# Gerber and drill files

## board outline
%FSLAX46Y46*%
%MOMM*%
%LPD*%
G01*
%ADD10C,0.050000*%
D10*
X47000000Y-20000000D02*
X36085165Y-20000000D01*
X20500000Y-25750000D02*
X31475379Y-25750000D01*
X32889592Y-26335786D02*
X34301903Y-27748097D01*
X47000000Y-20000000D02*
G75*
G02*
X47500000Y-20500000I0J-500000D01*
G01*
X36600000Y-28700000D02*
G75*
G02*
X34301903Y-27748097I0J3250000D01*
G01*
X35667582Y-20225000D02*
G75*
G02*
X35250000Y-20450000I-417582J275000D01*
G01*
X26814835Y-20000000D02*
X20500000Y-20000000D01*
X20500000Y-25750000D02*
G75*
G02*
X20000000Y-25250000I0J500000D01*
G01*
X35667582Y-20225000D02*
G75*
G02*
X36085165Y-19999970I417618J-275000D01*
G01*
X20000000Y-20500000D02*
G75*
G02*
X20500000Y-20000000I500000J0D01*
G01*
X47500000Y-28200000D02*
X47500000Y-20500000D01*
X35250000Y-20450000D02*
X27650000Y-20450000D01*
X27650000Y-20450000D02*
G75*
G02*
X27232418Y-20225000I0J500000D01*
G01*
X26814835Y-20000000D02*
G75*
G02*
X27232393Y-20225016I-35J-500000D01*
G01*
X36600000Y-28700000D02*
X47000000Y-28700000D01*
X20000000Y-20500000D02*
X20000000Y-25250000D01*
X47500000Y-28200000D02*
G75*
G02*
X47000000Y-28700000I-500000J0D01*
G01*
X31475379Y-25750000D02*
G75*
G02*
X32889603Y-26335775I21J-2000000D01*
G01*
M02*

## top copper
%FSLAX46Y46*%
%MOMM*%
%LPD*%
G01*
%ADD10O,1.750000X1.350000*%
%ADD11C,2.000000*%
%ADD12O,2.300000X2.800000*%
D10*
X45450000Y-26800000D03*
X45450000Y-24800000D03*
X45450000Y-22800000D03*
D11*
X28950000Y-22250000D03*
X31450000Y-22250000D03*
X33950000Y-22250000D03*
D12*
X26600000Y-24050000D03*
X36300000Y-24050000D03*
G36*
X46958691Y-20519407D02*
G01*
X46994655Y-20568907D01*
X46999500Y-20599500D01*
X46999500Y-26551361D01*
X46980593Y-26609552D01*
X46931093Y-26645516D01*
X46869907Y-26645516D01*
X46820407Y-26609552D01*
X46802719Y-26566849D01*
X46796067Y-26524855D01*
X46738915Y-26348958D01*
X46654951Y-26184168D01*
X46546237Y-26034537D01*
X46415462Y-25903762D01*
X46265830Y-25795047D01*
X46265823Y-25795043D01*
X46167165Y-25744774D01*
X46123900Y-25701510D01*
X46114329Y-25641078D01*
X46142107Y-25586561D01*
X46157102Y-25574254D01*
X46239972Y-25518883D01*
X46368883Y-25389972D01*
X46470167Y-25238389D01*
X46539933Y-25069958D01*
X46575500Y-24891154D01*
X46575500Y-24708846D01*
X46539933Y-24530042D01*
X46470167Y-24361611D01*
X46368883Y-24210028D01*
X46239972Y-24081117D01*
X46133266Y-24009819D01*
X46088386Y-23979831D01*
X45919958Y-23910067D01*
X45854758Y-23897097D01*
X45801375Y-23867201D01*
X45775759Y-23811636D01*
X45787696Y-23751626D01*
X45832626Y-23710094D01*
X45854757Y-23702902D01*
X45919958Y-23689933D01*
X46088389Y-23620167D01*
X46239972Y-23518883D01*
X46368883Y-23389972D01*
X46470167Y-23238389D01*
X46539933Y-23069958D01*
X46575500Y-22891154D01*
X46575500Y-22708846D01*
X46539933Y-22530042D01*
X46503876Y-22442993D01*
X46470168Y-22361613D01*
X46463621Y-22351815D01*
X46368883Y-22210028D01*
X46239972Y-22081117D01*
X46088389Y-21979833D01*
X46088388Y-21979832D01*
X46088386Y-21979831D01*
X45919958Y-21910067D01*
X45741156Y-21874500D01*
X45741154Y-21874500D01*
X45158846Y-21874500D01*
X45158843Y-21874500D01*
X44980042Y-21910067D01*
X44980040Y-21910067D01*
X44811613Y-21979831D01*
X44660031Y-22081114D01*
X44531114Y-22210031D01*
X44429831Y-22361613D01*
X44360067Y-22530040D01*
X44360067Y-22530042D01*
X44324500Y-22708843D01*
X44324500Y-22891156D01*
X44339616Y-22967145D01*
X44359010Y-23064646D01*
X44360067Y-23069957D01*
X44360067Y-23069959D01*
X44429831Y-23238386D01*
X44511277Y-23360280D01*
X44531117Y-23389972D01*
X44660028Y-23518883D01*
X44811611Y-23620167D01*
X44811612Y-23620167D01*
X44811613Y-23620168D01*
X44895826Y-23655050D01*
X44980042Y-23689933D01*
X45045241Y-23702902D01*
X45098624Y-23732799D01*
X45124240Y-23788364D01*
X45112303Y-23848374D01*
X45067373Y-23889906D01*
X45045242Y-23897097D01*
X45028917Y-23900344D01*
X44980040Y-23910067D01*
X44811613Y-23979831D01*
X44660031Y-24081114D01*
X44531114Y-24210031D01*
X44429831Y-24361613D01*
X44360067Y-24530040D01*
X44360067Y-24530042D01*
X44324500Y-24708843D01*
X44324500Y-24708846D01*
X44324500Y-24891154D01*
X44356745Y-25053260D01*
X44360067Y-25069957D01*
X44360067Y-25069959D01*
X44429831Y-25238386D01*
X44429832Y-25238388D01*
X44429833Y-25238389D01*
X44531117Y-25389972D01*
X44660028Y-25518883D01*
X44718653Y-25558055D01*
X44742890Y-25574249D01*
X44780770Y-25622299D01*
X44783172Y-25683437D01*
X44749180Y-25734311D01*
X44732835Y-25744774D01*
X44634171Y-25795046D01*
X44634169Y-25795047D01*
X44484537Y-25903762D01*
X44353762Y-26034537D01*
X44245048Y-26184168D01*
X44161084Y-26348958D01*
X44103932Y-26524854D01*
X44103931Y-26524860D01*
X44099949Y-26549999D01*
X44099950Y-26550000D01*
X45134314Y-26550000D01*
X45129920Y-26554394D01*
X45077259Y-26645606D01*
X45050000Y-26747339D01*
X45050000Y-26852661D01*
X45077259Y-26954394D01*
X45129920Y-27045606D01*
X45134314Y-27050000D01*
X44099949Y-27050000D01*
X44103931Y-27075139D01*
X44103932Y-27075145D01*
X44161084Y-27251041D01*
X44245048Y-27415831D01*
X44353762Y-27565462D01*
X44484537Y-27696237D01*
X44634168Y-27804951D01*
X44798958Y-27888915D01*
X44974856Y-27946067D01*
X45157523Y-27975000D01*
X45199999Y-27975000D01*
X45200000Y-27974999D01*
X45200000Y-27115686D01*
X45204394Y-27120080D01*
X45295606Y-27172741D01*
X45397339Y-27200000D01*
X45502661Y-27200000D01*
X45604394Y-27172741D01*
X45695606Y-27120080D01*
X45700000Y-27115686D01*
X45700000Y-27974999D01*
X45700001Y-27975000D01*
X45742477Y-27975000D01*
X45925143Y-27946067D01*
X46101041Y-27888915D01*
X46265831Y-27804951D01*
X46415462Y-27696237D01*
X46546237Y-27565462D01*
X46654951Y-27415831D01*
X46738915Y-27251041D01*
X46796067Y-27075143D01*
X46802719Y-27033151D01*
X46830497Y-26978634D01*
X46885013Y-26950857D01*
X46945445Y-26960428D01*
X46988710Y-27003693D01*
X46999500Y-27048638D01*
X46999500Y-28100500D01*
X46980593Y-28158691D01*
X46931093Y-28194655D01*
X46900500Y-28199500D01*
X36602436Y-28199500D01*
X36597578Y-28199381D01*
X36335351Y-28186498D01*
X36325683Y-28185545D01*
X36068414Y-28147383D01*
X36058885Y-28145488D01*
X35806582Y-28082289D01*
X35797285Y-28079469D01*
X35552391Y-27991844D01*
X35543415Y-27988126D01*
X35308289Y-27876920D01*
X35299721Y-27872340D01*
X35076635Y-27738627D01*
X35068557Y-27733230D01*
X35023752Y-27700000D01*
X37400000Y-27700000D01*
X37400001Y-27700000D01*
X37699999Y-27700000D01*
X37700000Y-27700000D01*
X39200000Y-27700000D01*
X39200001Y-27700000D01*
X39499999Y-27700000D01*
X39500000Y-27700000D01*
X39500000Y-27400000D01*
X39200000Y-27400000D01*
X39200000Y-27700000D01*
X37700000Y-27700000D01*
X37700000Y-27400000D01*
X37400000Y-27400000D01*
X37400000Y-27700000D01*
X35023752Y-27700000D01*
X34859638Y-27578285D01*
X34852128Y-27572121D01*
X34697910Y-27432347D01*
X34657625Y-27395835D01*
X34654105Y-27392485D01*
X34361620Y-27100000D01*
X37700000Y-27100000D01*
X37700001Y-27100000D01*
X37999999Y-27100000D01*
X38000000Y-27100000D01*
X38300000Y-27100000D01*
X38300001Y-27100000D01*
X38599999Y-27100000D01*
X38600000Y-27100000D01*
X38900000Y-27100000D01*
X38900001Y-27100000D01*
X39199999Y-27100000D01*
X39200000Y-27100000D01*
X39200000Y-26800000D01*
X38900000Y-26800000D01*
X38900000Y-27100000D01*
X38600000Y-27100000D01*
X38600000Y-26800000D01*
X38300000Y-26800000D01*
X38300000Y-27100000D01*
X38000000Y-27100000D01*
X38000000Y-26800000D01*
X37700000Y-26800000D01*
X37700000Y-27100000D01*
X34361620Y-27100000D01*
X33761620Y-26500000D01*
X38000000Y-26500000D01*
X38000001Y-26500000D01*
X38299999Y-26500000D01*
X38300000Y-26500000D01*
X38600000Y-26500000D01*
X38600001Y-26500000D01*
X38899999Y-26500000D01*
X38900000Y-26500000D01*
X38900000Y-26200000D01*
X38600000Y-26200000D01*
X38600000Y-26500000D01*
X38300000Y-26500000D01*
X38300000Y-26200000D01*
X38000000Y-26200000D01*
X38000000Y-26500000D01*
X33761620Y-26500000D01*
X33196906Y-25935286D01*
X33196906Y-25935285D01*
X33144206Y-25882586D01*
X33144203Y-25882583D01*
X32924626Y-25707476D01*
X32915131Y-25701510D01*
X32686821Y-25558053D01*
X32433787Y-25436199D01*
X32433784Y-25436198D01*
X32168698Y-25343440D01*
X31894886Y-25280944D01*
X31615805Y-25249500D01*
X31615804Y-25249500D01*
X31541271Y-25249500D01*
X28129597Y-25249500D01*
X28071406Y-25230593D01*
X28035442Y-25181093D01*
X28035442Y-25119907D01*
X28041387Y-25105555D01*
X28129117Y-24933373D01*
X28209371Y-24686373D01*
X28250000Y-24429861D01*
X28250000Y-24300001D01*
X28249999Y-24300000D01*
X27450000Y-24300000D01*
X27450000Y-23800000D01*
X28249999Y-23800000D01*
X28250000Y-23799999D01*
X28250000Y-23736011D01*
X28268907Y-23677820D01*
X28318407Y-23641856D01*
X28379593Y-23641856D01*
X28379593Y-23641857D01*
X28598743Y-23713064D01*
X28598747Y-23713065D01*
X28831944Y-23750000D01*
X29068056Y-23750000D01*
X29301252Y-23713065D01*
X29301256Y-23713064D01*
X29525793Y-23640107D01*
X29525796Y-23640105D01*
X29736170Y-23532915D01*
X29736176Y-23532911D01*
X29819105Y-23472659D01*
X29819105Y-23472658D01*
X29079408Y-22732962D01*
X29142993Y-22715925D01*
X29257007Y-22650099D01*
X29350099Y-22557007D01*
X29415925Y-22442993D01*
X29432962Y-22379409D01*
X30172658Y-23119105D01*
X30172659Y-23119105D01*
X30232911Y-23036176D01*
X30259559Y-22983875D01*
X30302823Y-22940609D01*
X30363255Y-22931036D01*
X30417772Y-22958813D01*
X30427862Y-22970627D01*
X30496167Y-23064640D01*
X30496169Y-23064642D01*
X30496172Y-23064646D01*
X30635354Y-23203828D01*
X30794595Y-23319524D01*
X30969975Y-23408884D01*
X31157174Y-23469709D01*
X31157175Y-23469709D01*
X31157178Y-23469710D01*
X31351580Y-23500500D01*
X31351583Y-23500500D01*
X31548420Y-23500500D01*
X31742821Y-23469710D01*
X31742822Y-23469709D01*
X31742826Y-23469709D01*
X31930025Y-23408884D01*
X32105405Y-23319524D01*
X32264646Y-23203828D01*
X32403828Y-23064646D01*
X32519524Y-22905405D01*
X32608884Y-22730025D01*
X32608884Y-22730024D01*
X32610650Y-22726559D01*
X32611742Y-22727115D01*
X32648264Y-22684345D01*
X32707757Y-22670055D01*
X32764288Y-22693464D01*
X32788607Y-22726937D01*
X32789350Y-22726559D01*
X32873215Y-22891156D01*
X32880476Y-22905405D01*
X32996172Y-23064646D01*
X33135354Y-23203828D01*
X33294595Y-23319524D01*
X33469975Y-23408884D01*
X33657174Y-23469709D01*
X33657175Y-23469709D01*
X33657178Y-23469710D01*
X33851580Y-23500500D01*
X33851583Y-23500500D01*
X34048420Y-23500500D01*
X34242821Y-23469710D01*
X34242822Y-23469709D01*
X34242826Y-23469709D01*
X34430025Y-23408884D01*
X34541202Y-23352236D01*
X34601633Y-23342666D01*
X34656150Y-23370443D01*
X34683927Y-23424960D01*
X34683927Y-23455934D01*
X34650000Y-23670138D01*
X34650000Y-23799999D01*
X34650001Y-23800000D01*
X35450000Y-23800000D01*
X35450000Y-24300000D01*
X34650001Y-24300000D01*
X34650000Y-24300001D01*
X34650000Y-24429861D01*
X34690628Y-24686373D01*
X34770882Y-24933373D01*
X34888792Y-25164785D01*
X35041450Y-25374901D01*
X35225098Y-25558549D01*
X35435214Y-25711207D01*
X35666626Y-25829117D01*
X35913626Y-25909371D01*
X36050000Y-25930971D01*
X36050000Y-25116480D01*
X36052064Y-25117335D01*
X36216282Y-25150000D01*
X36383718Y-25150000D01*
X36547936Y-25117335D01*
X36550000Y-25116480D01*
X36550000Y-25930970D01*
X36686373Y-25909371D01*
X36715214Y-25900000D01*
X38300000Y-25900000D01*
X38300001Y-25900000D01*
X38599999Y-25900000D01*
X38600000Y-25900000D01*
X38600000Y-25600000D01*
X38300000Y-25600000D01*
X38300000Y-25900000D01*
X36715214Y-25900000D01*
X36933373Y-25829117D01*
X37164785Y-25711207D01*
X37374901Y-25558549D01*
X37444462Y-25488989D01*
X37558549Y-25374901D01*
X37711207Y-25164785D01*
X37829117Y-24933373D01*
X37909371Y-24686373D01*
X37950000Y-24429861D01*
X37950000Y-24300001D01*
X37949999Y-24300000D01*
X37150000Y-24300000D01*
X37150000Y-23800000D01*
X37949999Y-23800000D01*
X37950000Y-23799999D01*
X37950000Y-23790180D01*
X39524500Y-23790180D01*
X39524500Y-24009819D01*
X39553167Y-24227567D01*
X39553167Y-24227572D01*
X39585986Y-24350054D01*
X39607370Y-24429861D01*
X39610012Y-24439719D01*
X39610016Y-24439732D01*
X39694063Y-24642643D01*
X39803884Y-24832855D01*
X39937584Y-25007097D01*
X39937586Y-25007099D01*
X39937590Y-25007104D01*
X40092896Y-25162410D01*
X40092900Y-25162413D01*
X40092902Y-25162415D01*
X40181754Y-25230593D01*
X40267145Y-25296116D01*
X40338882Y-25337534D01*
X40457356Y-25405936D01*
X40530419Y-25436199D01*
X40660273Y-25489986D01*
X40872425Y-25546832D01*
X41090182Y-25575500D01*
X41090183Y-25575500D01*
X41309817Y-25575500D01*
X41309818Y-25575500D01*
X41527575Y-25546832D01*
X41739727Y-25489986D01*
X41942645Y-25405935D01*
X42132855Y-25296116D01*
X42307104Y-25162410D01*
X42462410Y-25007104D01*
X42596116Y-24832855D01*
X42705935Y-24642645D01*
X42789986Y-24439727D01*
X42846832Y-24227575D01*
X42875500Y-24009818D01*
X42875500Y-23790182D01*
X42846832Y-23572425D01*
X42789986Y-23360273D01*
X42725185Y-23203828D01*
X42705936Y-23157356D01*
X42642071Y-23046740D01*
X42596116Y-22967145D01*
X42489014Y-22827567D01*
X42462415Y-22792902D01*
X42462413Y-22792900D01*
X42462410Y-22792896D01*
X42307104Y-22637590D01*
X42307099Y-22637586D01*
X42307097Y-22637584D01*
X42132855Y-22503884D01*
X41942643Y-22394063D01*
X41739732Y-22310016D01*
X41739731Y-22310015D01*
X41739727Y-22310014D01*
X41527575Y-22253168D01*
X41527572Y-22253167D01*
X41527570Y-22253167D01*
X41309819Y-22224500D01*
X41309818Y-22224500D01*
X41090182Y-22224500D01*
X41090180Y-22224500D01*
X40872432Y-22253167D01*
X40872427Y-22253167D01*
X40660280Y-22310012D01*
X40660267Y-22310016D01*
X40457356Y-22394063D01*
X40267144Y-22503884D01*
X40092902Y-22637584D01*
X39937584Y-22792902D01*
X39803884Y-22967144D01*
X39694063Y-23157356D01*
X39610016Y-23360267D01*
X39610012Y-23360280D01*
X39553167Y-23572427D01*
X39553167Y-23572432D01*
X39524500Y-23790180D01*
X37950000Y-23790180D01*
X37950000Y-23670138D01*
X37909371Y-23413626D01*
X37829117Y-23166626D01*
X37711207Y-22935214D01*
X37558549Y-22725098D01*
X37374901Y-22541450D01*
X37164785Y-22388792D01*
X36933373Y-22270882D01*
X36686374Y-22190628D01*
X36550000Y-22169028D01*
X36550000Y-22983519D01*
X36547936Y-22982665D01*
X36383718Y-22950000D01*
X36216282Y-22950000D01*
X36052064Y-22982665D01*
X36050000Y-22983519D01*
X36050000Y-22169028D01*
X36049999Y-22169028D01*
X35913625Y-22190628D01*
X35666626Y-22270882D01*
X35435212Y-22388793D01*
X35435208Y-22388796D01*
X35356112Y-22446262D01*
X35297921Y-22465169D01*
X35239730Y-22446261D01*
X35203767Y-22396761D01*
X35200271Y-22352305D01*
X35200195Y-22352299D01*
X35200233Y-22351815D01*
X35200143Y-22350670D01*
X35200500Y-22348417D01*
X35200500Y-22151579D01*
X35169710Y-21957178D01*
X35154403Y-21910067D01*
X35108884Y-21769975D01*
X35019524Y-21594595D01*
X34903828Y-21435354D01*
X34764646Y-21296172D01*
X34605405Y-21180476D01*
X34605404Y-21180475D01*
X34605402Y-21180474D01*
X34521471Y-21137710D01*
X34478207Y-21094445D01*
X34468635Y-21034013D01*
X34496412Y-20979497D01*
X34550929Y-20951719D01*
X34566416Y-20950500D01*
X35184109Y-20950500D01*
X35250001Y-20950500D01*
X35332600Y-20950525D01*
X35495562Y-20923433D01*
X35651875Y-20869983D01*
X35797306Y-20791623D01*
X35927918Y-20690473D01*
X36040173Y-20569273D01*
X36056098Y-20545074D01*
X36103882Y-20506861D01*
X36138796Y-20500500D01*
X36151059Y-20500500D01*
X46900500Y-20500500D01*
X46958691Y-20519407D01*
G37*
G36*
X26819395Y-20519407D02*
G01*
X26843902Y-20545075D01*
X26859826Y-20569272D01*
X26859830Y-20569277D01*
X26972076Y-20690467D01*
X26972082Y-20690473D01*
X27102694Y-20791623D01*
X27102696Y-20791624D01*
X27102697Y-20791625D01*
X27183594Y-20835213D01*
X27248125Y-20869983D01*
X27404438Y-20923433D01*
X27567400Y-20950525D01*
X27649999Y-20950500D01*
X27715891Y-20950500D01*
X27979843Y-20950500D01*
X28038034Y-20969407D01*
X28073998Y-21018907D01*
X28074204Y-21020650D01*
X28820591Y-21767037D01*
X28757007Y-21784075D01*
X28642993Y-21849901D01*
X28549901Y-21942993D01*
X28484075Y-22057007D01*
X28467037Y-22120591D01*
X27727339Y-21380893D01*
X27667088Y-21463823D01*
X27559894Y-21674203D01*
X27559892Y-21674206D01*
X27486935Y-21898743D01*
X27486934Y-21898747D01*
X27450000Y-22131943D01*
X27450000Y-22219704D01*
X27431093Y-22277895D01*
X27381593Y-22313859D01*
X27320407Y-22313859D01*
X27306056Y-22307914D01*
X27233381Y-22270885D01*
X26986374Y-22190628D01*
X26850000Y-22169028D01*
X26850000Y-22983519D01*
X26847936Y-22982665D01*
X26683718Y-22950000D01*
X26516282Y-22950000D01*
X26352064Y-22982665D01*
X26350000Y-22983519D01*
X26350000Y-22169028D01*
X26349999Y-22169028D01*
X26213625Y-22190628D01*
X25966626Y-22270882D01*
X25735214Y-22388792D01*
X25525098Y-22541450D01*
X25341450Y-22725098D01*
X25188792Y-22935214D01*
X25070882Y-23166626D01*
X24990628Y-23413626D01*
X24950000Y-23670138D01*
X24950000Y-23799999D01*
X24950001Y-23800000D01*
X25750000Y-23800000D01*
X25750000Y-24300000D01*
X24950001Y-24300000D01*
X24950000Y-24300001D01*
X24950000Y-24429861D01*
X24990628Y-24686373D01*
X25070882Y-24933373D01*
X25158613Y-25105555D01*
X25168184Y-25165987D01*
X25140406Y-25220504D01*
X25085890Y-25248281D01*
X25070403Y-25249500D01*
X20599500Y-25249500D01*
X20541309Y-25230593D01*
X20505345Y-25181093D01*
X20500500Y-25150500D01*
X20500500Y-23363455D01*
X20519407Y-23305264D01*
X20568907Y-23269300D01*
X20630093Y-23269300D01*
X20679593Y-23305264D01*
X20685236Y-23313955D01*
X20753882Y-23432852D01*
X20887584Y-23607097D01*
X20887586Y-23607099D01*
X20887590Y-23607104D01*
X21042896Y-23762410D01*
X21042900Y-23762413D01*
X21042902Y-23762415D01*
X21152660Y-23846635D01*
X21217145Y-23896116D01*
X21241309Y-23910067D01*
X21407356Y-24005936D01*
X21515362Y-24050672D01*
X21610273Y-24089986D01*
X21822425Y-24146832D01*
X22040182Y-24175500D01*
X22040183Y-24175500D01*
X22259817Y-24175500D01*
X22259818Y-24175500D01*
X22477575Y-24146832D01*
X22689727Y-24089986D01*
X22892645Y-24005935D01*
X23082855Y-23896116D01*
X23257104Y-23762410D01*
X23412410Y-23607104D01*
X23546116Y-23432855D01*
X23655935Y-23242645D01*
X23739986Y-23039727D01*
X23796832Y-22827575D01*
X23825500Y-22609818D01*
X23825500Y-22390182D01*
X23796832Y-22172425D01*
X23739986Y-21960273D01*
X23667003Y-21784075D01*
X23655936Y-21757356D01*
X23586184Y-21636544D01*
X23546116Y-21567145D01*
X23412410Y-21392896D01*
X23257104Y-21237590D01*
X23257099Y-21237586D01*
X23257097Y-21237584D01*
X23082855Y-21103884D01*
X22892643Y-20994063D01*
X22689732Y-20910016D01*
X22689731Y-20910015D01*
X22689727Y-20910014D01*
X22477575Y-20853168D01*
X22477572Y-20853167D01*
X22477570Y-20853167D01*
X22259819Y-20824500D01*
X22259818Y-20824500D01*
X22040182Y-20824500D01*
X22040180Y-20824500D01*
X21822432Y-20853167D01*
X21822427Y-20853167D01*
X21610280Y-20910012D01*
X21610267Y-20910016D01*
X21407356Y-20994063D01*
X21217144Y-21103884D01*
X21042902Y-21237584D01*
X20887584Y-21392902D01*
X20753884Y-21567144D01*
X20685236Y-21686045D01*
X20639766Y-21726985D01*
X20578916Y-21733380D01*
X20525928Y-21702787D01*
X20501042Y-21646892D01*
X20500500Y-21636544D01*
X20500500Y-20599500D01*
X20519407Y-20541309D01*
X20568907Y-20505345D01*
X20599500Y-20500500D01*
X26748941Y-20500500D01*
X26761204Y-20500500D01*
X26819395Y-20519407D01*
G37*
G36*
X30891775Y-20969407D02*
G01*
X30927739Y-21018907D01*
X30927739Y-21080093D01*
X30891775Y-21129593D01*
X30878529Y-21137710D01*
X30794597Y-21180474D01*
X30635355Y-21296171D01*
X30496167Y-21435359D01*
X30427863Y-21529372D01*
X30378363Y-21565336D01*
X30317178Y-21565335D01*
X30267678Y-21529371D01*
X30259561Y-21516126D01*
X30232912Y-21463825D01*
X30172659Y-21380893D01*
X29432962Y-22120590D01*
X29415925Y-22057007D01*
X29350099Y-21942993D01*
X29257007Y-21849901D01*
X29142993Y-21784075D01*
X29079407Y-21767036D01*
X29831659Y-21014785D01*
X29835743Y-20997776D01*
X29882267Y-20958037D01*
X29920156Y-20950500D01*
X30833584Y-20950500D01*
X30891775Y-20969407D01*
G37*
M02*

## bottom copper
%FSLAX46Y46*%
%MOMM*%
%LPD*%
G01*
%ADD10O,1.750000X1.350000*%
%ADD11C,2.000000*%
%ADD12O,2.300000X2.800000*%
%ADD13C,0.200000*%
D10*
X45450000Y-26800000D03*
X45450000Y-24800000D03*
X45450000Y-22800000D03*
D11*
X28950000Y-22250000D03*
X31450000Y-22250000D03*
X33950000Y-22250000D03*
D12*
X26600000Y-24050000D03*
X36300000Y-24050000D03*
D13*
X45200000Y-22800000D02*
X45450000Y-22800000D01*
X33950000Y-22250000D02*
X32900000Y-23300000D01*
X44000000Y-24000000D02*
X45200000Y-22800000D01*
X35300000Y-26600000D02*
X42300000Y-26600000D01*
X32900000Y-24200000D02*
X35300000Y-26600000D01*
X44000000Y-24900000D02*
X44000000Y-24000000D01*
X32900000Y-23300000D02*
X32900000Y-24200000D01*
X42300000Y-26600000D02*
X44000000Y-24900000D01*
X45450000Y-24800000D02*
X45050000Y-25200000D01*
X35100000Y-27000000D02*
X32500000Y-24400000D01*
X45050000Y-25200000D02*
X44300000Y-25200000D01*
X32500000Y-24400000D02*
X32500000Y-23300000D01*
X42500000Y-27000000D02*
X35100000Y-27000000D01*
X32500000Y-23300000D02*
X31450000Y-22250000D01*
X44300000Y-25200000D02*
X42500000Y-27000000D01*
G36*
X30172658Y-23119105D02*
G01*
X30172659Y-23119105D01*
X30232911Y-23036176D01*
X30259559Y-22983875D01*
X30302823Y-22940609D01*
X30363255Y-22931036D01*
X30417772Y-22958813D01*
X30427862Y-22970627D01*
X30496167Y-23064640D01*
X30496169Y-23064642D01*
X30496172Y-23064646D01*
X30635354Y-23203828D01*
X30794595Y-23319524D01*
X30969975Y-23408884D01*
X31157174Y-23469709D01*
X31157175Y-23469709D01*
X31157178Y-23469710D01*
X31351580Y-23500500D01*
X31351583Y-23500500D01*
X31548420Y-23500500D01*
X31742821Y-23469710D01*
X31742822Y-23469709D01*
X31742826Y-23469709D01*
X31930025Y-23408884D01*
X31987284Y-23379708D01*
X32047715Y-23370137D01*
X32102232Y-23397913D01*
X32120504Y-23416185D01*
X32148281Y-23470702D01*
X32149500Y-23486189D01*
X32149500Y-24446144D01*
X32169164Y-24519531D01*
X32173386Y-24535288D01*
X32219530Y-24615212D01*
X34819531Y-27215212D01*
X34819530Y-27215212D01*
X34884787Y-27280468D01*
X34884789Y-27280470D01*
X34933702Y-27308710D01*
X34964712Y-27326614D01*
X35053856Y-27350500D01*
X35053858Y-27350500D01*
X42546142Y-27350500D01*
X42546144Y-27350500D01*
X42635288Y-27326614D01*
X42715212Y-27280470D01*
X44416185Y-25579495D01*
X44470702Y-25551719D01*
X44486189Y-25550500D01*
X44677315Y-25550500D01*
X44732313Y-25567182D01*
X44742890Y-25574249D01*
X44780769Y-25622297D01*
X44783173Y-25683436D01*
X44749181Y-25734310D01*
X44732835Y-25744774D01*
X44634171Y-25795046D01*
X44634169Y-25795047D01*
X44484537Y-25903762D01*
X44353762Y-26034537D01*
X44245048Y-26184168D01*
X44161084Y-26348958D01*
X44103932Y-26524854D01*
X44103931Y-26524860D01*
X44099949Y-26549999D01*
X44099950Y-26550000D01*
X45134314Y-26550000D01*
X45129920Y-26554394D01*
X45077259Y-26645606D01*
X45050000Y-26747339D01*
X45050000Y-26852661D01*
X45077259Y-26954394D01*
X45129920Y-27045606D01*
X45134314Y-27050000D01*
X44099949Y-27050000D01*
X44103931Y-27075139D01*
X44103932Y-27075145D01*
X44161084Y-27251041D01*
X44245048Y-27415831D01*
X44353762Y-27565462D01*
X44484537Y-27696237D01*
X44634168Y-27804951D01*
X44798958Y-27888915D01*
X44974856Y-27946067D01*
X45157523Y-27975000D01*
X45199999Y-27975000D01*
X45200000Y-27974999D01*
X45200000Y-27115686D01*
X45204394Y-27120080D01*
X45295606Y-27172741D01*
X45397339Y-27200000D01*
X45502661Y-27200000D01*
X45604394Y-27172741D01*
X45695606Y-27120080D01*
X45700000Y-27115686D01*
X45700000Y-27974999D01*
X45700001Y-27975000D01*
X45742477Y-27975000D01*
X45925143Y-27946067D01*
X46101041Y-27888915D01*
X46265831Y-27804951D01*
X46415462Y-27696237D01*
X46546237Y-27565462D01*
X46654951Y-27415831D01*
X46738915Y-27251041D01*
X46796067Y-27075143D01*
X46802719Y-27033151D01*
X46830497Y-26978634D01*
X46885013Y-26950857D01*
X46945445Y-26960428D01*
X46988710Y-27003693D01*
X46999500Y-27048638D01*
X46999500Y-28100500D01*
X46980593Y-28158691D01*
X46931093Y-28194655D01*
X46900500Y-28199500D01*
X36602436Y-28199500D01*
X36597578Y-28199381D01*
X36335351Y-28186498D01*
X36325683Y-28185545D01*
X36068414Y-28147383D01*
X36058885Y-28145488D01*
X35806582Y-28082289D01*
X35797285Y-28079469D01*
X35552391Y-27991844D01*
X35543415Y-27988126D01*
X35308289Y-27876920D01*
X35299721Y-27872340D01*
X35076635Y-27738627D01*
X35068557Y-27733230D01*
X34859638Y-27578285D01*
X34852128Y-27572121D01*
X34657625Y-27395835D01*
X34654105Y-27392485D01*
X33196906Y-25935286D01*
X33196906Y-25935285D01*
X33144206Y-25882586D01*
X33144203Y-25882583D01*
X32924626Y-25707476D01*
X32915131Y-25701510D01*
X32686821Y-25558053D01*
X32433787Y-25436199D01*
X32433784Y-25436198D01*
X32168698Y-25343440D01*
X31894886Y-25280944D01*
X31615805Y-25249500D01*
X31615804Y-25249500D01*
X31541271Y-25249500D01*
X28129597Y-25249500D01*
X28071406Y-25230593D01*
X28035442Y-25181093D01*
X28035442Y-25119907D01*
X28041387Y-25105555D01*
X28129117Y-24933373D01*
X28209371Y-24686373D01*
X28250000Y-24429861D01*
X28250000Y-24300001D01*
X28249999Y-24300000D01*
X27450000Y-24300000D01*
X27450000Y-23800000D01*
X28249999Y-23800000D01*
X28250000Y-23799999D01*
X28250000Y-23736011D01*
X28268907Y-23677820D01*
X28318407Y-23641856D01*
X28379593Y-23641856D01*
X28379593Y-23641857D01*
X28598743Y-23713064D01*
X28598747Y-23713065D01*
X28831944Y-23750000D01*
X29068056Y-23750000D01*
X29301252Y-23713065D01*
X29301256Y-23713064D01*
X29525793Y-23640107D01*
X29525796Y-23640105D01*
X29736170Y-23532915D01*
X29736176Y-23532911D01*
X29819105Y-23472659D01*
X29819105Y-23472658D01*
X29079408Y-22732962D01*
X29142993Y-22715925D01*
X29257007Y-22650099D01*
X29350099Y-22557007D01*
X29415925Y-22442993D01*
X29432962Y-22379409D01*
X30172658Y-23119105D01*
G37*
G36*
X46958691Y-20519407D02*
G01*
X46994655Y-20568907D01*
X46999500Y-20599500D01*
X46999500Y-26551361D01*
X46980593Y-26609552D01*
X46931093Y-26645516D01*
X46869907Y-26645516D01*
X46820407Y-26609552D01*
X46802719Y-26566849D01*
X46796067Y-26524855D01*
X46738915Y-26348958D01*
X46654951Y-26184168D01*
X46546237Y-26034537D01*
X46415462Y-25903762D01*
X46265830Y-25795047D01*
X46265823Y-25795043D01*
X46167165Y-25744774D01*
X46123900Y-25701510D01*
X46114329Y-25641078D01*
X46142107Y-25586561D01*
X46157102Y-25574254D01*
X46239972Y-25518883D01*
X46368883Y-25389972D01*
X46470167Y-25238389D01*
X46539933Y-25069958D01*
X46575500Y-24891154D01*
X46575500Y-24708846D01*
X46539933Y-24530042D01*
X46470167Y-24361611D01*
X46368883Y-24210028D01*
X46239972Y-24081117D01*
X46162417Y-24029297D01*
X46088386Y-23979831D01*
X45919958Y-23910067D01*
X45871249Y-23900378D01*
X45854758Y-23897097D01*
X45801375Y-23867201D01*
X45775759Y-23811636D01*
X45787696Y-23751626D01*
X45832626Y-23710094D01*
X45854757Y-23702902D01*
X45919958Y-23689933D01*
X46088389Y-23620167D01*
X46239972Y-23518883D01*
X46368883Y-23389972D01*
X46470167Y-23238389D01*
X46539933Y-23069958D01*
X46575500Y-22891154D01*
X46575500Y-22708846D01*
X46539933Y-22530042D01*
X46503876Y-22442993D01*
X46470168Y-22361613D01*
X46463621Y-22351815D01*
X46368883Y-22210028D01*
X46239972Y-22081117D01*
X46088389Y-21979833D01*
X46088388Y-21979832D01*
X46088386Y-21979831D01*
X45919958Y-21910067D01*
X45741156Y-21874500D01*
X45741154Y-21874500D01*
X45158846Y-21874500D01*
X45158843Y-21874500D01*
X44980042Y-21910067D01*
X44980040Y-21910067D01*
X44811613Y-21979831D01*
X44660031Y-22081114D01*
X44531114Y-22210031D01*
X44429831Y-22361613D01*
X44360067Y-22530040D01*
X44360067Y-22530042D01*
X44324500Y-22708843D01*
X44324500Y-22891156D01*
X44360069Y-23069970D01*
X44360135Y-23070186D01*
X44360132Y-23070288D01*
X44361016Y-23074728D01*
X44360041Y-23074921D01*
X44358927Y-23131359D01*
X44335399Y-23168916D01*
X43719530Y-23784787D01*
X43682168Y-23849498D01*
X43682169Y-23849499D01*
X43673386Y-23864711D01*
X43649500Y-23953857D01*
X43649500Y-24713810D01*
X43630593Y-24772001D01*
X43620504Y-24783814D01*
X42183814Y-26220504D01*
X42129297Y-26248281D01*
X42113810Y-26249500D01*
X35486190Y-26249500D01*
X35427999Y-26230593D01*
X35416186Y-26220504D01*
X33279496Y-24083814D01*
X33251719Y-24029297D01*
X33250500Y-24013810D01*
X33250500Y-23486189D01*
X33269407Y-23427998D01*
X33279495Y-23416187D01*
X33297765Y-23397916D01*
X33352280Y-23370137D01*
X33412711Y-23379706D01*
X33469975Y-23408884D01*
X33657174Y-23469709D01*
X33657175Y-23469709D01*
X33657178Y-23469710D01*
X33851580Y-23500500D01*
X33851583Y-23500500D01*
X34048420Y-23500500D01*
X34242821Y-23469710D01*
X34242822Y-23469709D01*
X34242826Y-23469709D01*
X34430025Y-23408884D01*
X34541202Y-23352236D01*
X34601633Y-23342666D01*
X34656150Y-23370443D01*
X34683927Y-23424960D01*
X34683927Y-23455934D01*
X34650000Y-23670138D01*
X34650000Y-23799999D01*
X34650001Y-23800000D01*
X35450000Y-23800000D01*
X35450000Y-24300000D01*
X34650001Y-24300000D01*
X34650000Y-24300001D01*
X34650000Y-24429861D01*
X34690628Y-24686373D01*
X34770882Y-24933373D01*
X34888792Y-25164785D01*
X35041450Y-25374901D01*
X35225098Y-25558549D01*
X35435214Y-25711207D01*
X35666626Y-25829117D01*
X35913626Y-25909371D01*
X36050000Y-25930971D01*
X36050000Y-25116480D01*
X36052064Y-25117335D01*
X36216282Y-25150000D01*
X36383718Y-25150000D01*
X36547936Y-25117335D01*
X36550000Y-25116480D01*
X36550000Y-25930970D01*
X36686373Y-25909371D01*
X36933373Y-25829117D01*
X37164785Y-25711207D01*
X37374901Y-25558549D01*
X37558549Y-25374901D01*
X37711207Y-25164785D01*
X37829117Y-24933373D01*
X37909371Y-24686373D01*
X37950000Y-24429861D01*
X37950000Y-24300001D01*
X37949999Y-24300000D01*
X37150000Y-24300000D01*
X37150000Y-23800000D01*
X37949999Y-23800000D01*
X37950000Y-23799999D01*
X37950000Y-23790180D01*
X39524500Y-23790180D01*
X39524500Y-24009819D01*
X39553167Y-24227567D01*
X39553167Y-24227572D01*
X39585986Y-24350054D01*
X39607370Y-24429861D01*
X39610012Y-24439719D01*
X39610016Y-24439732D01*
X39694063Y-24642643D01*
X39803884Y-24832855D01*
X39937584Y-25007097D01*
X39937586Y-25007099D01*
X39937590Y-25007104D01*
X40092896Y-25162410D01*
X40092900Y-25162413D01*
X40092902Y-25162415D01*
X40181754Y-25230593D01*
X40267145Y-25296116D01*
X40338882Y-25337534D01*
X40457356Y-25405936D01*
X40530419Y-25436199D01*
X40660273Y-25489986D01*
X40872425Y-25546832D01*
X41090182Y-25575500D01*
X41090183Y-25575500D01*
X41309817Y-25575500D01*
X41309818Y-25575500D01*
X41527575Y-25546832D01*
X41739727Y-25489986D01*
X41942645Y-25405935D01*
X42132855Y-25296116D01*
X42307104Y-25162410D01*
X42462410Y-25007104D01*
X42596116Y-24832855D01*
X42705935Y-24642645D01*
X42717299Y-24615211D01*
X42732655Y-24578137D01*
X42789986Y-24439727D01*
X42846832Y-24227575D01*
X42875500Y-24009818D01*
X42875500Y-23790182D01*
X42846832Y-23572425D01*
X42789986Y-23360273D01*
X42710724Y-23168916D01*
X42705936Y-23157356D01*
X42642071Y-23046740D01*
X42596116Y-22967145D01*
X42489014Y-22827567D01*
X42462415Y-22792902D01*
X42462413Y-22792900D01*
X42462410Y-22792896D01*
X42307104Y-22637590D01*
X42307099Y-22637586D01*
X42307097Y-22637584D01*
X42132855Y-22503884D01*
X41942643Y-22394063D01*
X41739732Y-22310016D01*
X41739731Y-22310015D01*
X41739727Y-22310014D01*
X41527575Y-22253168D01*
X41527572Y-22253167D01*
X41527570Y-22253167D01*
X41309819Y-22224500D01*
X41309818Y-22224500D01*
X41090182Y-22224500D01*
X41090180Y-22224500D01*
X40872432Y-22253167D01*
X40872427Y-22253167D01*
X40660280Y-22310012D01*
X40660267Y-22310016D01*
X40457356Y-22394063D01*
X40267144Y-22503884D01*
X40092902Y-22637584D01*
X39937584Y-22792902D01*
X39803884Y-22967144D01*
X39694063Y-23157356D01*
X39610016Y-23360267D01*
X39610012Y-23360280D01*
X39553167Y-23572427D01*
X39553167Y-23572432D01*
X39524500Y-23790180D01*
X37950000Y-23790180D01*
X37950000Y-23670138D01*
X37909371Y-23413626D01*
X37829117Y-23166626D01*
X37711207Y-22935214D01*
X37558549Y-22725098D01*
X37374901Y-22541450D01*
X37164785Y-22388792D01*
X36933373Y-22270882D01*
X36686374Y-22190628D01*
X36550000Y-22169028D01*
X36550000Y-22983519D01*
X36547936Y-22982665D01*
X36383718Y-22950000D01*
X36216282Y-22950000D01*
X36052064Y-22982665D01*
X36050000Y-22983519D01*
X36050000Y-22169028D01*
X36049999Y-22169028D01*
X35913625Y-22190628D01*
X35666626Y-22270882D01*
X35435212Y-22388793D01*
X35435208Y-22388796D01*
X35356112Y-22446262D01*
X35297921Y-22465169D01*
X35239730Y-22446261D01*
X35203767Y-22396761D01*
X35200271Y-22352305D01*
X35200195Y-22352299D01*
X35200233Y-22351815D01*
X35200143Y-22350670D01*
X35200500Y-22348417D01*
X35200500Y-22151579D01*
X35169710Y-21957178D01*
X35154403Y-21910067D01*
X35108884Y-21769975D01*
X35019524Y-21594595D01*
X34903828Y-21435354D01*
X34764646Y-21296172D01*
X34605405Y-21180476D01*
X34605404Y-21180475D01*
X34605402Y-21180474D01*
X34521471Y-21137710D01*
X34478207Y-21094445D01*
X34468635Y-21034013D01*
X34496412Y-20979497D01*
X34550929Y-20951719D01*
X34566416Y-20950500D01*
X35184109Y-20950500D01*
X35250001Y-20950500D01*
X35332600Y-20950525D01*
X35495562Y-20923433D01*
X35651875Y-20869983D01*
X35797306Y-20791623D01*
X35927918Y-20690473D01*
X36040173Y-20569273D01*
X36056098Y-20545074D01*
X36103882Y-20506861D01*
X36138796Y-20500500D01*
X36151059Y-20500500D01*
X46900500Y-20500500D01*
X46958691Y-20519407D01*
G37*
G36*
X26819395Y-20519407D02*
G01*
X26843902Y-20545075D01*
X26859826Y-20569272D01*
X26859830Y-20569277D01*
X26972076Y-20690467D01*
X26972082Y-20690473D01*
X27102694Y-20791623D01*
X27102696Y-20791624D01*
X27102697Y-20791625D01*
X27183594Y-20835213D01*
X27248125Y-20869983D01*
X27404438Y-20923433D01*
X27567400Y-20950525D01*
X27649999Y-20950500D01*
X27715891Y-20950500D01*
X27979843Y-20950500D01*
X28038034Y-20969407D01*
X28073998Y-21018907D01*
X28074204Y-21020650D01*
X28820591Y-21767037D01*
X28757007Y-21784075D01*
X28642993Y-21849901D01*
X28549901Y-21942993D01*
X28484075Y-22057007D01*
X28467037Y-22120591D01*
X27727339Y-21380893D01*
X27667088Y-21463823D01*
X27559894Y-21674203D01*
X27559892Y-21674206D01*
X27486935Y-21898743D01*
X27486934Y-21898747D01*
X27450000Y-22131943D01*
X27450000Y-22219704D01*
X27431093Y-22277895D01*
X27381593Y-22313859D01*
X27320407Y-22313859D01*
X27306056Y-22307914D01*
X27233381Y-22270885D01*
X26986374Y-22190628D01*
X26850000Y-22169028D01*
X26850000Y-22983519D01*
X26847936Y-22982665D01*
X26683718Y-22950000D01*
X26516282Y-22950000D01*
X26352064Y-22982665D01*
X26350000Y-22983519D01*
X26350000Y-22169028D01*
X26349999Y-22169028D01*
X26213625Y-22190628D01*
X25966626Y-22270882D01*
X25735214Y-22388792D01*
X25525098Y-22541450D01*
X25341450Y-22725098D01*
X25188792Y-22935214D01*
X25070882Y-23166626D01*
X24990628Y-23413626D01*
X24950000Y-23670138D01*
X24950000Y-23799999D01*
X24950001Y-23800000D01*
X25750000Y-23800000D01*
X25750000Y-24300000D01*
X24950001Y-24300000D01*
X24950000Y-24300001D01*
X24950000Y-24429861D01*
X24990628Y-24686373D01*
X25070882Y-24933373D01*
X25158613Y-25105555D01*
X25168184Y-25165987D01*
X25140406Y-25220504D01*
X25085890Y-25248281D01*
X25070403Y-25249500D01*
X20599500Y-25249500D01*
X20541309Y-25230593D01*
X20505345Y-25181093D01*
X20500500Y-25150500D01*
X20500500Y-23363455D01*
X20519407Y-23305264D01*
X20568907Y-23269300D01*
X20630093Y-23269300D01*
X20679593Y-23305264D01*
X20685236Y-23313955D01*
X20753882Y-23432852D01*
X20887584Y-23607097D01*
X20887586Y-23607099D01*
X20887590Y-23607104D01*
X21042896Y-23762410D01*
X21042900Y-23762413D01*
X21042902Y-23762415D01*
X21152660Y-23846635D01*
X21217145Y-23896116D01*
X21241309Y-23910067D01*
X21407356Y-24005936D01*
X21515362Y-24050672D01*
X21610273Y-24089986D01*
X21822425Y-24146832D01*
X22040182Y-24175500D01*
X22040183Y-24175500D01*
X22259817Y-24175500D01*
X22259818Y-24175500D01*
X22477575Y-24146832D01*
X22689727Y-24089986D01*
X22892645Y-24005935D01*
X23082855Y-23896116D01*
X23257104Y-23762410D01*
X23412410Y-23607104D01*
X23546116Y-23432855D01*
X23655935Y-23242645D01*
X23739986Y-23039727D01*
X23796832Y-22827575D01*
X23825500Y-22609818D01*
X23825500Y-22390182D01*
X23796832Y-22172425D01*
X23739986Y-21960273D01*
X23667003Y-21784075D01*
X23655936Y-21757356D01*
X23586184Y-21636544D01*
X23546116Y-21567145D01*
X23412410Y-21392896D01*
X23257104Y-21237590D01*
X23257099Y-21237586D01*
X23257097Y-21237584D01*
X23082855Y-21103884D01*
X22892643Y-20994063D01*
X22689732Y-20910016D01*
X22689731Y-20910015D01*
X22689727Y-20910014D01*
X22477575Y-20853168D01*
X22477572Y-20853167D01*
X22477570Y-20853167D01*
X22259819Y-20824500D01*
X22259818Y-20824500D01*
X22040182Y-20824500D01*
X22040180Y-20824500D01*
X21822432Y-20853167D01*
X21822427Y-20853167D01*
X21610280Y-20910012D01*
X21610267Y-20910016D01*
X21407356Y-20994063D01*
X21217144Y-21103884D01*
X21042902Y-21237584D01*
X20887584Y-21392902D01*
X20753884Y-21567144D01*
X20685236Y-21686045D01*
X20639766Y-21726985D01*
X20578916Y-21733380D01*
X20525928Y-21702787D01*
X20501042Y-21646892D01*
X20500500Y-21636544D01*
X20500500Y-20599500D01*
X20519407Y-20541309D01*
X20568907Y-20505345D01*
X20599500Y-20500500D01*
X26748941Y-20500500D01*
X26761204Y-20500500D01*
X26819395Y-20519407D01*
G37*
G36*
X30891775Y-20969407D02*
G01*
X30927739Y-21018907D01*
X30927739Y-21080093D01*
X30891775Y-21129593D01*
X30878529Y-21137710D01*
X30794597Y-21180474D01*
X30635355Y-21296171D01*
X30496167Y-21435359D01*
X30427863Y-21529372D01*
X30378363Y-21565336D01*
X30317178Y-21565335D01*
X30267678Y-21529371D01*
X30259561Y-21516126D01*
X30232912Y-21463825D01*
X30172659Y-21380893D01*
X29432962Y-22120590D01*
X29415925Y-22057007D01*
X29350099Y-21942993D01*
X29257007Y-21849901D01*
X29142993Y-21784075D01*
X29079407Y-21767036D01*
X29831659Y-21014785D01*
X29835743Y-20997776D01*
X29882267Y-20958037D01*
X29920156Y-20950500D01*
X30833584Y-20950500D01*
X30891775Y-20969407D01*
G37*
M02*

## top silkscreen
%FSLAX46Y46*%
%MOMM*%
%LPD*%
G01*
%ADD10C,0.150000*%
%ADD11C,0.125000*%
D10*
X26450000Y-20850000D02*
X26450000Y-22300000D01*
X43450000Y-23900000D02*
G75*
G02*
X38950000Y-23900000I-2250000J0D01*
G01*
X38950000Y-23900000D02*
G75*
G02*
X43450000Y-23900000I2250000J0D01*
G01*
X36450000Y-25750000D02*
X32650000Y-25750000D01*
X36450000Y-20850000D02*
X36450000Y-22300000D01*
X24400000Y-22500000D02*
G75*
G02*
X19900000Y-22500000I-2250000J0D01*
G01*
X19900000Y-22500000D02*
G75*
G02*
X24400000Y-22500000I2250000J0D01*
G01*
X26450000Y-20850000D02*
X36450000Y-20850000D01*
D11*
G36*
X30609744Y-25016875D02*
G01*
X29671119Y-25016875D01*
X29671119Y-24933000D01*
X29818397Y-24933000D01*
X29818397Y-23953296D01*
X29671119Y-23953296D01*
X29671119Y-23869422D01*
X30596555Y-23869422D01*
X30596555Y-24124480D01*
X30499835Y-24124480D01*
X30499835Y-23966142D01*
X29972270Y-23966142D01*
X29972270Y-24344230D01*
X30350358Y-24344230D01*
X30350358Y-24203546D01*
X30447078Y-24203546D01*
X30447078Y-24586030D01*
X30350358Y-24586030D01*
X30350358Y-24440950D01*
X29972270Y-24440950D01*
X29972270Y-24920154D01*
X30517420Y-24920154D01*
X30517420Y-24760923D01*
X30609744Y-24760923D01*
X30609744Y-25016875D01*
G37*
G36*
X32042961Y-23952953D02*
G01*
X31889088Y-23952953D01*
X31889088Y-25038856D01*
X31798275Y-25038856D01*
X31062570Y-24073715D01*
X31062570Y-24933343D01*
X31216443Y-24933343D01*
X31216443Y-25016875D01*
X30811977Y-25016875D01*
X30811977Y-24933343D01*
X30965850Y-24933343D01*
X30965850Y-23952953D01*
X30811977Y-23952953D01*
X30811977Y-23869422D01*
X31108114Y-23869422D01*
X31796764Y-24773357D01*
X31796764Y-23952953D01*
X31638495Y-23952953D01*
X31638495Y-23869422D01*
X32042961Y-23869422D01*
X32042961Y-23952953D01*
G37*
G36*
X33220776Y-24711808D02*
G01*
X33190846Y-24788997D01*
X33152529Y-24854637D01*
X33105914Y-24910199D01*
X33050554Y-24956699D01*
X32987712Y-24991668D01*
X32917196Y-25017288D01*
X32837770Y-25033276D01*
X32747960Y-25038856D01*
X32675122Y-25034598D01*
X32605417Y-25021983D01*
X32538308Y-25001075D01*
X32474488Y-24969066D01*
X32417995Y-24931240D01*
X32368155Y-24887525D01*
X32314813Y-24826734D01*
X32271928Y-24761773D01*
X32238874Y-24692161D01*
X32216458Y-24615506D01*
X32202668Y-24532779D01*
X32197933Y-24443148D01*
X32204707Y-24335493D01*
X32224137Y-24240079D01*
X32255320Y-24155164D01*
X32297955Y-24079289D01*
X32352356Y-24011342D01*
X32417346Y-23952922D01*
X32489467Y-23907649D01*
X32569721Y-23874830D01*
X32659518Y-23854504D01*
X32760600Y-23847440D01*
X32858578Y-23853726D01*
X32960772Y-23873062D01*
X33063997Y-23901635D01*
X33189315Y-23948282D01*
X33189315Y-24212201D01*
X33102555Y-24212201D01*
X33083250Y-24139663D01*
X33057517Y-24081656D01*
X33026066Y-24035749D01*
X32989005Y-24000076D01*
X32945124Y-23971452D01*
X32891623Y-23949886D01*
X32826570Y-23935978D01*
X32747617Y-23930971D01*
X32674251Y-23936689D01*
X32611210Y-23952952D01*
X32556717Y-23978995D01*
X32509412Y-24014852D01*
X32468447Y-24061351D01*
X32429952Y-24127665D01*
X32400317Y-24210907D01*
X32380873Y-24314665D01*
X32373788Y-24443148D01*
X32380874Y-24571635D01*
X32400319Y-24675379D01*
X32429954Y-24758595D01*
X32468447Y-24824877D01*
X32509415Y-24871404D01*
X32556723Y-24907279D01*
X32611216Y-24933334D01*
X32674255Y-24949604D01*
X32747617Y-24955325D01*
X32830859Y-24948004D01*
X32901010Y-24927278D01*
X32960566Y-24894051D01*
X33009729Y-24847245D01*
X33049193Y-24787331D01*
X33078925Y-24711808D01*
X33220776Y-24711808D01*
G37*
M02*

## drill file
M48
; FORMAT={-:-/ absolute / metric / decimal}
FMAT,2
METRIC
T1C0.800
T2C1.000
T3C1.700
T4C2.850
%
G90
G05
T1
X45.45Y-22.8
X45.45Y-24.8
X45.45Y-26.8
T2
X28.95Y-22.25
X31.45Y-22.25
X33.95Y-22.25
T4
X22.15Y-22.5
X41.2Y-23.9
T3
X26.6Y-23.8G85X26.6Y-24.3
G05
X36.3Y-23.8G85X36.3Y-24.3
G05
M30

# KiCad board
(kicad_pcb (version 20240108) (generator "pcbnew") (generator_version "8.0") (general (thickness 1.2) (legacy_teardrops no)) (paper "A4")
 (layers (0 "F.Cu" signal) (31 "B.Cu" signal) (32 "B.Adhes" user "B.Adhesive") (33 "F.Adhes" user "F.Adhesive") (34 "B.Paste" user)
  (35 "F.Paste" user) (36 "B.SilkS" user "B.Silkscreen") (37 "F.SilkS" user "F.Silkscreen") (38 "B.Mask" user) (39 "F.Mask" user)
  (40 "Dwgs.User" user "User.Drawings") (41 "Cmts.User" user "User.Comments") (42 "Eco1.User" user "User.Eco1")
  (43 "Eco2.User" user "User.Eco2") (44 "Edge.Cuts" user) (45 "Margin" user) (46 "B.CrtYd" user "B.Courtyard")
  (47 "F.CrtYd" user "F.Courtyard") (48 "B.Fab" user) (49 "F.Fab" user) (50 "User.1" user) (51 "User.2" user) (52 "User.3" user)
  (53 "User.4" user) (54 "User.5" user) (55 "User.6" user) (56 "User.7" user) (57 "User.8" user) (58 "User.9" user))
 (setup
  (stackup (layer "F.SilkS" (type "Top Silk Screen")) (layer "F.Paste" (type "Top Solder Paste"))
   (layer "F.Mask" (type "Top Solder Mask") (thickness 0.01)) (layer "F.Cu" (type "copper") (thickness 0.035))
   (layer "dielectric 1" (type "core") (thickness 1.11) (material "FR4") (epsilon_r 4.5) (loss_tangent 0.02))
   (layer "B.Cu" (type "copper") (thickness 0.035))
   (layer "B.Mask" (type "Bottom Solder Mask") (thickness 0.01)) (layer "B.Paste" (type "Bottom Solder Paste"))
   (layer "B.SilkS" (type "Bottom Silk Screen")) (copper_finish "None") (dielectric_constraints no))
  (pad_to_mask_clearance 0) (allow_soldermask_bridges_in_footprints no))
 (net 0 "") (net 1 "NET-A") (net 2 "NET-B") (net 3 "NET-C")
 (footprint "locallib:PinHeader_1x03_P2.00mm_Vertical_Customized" (layer "F.Cu") (at 45.45 26.8 180)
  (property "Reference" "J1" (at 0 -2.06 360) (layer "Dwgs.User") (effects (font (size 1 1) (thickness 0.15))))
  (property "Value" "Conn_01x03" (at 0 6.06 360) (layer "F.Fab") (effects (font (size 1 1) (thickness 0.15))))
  (pad "1" thru_hole oval (at 0 0 180) (size 1.75 1.35) (drill 0.8) (layers "*.Cu" "F.Mask") (remove_unused_layers no) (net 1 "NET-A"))
  (pad "2" thru_hole oval (at 0 2 180) (size 1.75 1.35) (drill 0.8) (layers "*.Cu" "F.Mask") (remove_unused_layers no) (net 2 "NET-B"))
  (pad "3" thru_hole oval (at 0 4 180) (size 1.75 1.35) (drill 0.8) (layers "*.Cu" "F.Mask") (remove_unused_layers no) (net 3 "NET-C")))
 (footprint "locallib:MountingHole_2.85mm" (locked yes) (layer "F.Cu") (at 22.15 22.5)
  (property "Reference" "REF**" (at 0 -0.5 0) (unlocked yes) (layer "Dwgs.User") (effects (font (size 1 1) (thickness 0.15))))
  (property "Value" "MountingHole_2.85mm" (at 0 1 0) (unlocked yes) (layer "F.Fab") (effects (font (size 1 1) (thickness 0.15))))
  (pad "" np_thru_hole circle (at 0 0) (size 2.85 2.85) (drill 2.85) (layers "F&B.Cu" "*.Mask")))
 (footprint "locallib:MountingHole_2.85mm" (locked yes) (layer "F.Cu") (at 41.2 23.9)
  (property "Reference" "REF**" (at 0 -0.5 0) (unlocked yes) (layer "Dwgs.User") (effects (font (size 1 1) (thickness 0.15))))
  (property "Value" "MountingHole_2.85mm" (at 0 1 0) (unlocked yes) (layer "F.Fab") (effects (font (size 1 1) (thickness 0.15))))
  (pad "" np_thru_hole circle (at 0 0) (size 2.85 2.85) (drill 2.85) (layers "F&B.Cu" "*.Mask")))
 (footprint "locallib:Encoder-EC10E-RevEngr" (layer "F.Cu") (at 31.45 22.25)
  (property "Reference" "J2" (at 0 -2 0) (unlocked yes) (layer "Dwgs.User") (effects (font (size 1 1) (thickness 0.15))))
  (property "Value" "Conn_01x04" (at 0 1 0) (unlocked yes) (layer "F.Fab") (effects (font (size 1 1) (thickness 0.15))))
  (pad "1" thru_hole circle (at -2.5 0) (size 2 2) (drill 1) (layers "*.Cu" "B.Mask") (remove_unused_layers no) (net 1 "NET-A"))
  (pad "2" thru_hole circle (at 0 0) (size 2 2) (drill 1) (layers "*.Cu" "B.Mask") (remove_unused_layers no) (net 2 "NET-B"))
  (pad "3" thru_hole circle (at 2.5 0) (size 2 2) (drill 1) (layers "*.Cu" "B.Mask") (remove_unused_layers no) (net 3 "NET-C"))
  (pad "4" thru_hole oval (at -4.85 1.8) (size 2.3 2.8) (drill oval 1.7 2.2) (layers "*.Cu" "*.Mask") (remove_unused_layers no)
   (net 1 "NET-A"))
  (pad "4" thru_hole oval (at 4.85 1.8) (size 2.3 2.8) (drill oval 1.7 2.2) (layers "*.Cu" "*.Mask") (remove_unused_layers no)
   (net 1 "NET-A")))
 (gr_line (start 26.45 20.85) (end 26.45 22.3) (stroke (width 0.15) (type default)) (layer "F.SilkS"))
 (gr_circle (center 41.2 23.9) (end 43.45 23.9) (stroke (width 0.15) (type default)) (fill none) (layer "F.SilkS"))
 (gr_line (start 36.45 25.75) (end 32.65 25.75) (stroke (width 0.15) (type default)) (layer "F.SilkS"))
 (gr_line (start 36.45 20.85) (end 36.45 22.3) (stroke (width 0.15) (type default)) (layer "F.SilkS"))
 (gr_circle (center 22.15 22.5) (end 24.4 22.5) (stroke (width 0.15) (type default)) (fill none) (layer "F.SilkS"))
 (gr_line (start 26.45 20.85) (end 36.45 20.85) (stroke (width 0.15) (type default)) (layer "F.SilkS"))
 (gr_line (start 47 20) (end 36.085165 20) (stroke (width 0.05) (type default)) (layer "Edge.Cuts"))
 (gr_line (start 20.5 25.75) (end 31.475379 25.75) (stroke (width 0.05) (type default)) (layer "Edge.Cuts"))
 (gr_line (start 32.889592 26.335786) (end 34.301903 27.748097) (stroke (width 0.05) (type default)) (layer "Edge.Cuts"))
 (gr_arc (start 47 20) (mid 47.353553 20.146447) (end 47.5 20.5) (stroke (width 0.05) (type default)) (layer "Edge.Cuts"))
 (gr_arc (start 36.6 28.7) (mid 35.356279 28.452608) (end 34.301903 27.748097) (stroke (width 0.05) (type default)) (layer "Edge.Cuts"))
 (gr_arc (start 35.667582 20.225) (mid 35.487171 20.39017) (end 35.25 20.45) (stroke (width 0.05) (type default)) (layer "Edge.Cuts"))
 (gr_line (start 26.814835 20) (end 20.5 20) (stroke (width 0.05) (type default)) (layer "Edge.Cuts"))
 (gr_arc (start 20.5 25.75) (mid 20.146447 25.603553) (end 20 25.25) (stroke (width 0.05) (type default)) (layer "Edge.Cuts"))
 (gr_arc (start 35.667582 20.225) (mid 35.847994 20.05983) (end 36.085165 20) (stroke (width 0.05) (type default)) (layer "Edge.Cuts"))
 (gr_arc (start 20 20.5) (mid 20.146447 20.146447) (end 20.5 20) (stroke (width 0.05) (type default)) (layer "Edge.Cuts"))
 (gr_line (start 47.5 28.2) (end 47.5 20.5) (stroke (width 0.05) (type default)) (layer "Edge.Cuts"))
 (gr_line (start 35.25 20.45) (end 27.65 20.45) (stroke (width 0.05) (type default)) (layer "Edge.Cuts"))
 (gr_arc (start 27.65 20.45) (mid 27.412829 20.39017) (end 27.232418 20.225) (stroke (width 0.05) (type default)) (layer "Edge.Cuts"))
 (gr_arc (start 26.814835 20) (mid 27.052006 20.05983) (end 27.232418 20.225) (stroke (width 0.05) (type default)) (layer "Edge.Cuts"))
 (gr_line (start 36.6 28.7) (end 47 28.7) (stroke (width 0.05) (type default)) (layer "Edge.Cuts"))
 (gr_line (start 20 20.5) (end 20 25.25) (stroke (width 0.05) (type default)) (layer "Edge.Cuts"))
 (gr_arc (start 47.5 28.2) (mid 47.353553 28.553553) (end 47 28.7) (stroke (width 0.05) (type default)) (layer "Edge.Cuts"))
 (gr_arc (start 31.475379 25.75) (mid 32.240746 25.902241) (end 32.889592 26.335786) (stroke (width 0.05) (type default))
  (layer "Edge.Cuts"))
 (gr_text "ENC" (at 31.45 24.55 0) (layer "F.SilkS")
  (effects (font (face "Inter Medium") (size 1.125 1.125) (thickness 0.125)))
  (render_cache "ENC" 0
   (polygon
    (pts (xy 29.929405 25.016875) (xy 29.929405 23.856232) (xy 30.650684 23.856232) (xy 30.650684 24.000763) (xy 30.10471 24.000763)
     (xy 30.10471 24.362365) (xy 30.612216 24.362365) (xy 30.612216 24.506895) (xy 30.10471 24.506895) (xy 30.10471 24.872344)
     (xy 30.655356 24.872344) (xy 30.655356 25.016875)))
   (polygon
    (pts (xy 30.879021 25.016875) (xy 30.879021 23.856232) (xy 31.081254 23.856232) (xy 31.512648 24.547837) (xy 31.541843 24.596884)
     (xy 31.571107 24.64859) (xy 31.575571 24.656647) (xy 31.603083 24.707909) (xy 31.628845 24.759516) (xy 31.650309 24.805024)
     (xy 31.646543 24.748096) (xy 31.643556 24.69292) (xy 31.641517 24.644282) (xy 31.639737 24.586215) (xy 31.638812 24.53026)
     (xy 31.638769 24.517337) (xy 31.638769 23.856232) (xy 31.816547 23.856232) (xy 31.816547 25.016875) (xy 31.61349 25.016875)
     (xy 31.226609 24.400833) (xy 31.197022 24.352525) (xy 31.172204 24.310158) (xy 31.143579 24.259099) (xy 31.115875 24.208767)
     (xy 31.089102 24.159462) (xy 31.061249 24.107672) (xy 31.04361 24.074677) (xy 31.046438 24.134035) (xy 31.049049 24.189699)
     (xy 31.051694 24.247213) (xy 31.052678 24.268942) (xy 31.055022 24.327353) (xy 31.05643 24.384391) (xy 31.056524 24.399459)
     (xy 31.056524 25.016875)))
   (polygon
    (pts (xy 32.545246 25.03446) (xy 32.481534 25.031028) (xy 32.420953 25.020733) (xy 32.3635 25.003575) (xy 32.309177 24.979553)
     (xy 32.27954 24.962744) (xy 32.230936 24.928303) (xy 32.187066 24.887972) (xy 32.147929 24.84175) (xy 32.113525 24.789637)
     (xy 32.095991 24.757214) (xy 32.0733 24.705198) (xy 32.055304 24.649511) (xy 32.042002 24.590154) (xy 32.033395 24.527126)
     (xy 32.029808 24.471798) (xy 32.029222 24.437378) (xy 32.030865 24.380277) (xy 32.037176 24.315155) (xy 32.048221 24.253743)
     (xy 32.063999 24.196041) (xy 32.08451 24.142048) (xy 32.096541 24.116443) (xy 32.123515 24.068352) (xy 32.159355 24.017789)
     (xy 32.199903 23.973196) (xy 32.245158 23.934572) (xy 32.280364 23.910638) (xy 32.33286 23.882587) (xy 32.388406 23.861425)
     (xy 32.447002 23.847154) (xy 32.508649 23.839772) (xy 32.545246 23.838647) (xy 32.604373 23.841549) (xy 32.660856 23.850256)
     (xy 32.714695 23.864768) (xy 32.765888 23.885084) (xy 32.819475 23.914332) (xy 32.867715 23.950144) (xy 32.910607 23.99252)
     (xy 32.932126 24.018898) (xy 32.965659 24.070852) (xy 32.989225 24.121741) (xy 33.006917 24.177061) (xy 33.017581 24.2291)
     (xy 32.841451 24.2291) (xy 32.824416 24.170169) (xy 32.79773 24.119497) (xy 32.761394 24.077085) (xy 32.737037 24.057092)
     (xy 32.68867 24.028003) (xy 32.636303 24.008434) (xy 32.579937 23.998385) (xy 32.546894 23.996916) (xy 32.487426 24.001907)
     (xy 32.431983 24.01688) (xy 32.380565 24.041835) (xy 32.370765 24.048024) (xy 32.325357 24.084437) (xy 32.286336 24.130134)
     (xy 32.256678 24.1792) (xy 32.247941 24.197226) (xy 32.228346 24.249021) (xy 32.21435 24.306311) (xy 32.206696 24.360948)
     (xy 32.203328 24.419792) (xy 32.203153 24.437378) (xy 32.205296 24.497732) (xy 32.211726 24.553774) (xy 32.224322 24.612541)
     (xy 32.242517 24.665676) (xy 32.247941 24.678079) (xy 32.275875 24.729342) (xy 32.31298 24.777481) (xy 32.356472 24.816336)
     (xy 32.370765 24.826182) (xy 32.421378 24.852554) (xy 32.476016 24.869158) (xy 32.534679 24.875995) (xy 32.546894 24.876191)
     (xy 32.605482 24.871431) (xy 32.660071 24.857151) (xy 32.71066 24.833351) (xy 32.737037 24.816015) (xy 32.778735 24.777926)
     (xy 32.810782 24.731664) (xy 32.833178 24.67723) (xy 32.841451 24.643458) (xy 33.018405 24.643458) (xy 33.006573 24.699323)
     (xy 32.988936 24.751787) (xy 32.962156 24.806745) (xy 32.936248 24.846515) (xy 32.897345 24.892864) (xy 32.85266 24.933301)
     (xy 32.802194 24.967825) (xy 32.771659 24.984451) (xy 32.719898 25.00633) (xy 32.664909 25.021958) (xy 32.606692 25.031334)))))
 (segment (start 45.2 22.8) (end 45.45 22.8) (width 0.2) (layer "B.Cu") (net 3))
 (segment (start 33.95 22.25) (end 32.9 23.3) (width 0.2) (layer "B.Cu") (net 3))
 (segment (start 44 24) (end 45.2 22.8) (width 0.2) (layer "B.Cu") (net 3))
 (segment (start 35.3 26.6) (end 42.3 26.6) (width 0.2) (layer "B.Cu") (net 3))
 (segment (start 32.9 24.2) (end 35.3 26.6) (width 0.2) (layer "B.Cu") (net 3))
 (segment (start 44 24.9) (end 44 24) (width 0.2) (layer "B.Cu") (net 3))
 (segment (start 32.9 23.3) (end 32.9 24.2) (width 0.2) (layer "B.Cu") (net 3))
 (segment (start 42.3 26.6) (end 44 24.9) (width 0.2) (layer "B.Cu") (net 3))
 (segment (start 45.45 24.8) (end 45.05 25.2) (width 0.2) (layer "B.Cu") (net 2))
 (segment (start 35.1 27) (end 32.5 24.4) (width 0.2) (layer "B.Cu") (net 2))
 (segment (start 45.05 25.2) (end 44.3 25.2) (width 0.2) (layer "B.Cu") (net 2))
 (segment (start 32.5 24.4) (end 32.5 23.3) (width 0.2) (layer "B.Cu") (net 2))
 (segment (start 42.5 27) (end 35.1 27) (width 0.2) (layer "B.Cu") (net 2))
 (segment (start 32.5 23.3) (end 31.45 22.25) (width 0.2) (layer "B.Cu") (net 2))
 (segment (start 44.3 25.2) (end 42.5 27) (width 0.2) (layer "B.Cu") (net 2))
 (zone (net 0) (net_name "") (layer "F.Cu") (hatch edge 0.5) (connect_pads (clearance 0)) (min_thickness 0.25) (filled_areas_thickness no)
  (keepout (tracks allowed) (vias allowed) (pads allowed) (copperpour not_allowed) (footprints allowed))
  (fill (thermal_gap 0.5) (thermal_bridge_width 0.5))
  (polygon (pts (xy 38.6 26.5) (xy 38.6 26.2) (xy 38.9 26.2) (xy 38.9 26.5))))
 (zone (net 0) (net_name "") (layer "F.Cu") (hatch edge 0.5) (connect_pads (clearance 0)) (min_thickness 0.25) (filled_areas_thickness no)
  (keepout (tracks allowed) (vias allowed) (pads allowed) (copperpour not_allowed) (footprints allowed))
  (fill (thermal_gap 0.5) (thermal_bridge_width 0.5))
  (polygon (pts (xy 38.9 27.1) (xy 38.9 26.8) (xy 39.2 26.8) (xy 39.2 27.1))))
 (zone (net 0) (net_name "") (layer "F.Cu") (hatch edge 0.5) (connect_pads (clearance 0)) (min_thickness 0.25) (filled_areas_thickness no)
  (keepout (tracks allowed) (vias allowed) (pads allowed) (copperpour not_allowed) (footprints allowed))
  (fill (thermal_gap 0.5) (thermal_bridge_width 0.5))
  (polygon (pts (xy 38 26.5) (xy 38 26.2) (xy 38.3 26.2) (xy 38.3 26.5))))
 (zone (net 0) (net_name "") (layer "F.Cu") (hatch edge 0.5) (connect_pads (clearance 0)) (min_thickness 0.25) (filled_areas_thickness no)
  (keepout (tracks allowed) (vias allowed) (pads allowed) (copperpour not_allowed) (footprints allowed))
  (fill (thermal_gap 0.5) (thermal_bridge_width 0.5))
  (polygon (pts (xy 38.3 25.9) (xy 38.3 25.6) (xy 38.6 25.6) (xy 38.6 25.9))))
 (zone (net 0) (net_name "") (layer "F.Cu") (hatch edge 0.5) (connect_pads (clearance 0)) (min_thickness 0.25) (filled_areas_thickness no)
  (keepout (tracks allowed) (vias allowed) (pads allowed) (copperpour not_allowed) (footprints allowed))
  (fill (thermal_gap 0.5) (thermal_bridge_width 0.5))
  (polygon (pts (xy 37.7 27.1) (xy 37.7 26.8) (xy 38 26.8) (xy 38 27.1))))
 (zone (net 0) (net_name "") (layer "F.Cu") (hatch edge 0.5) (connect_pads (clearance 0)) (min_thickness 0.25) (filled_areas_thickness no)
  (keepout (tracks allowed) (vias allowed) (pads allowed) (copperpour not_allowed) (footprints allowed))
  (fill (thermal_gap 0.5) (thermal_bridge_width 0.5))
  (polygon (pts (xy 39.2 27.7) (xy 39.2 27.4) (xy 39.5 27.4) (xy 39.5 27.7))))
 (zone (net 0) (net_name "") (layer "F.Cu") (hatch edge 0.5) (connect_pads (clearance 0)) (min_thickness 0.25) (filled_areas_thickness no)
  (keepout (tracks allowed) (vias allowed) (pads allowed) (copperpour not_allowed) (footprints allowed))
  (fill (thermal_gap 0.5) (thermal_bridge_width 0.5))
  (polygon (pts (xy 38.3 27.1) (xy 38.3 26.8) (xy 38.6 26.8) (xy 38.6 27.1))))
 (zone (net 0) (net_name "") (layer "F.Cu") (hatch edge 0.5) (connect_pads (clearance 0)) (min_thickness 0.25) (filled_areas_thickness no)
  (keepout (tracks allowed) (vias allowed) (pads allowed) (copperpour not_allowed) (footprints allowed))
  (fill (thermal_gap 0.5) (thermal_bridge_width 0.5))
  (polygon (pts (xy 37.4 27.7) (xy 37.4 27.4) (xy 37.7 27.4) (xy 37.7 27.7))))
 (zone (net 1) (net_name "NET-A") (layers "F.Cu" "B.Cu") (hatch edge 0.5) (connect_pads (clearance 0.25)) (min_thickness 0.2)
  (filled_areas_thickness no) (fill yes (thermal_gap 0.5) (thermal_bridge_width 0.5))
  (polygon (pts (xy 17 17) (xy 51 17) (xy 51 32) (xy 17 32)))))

